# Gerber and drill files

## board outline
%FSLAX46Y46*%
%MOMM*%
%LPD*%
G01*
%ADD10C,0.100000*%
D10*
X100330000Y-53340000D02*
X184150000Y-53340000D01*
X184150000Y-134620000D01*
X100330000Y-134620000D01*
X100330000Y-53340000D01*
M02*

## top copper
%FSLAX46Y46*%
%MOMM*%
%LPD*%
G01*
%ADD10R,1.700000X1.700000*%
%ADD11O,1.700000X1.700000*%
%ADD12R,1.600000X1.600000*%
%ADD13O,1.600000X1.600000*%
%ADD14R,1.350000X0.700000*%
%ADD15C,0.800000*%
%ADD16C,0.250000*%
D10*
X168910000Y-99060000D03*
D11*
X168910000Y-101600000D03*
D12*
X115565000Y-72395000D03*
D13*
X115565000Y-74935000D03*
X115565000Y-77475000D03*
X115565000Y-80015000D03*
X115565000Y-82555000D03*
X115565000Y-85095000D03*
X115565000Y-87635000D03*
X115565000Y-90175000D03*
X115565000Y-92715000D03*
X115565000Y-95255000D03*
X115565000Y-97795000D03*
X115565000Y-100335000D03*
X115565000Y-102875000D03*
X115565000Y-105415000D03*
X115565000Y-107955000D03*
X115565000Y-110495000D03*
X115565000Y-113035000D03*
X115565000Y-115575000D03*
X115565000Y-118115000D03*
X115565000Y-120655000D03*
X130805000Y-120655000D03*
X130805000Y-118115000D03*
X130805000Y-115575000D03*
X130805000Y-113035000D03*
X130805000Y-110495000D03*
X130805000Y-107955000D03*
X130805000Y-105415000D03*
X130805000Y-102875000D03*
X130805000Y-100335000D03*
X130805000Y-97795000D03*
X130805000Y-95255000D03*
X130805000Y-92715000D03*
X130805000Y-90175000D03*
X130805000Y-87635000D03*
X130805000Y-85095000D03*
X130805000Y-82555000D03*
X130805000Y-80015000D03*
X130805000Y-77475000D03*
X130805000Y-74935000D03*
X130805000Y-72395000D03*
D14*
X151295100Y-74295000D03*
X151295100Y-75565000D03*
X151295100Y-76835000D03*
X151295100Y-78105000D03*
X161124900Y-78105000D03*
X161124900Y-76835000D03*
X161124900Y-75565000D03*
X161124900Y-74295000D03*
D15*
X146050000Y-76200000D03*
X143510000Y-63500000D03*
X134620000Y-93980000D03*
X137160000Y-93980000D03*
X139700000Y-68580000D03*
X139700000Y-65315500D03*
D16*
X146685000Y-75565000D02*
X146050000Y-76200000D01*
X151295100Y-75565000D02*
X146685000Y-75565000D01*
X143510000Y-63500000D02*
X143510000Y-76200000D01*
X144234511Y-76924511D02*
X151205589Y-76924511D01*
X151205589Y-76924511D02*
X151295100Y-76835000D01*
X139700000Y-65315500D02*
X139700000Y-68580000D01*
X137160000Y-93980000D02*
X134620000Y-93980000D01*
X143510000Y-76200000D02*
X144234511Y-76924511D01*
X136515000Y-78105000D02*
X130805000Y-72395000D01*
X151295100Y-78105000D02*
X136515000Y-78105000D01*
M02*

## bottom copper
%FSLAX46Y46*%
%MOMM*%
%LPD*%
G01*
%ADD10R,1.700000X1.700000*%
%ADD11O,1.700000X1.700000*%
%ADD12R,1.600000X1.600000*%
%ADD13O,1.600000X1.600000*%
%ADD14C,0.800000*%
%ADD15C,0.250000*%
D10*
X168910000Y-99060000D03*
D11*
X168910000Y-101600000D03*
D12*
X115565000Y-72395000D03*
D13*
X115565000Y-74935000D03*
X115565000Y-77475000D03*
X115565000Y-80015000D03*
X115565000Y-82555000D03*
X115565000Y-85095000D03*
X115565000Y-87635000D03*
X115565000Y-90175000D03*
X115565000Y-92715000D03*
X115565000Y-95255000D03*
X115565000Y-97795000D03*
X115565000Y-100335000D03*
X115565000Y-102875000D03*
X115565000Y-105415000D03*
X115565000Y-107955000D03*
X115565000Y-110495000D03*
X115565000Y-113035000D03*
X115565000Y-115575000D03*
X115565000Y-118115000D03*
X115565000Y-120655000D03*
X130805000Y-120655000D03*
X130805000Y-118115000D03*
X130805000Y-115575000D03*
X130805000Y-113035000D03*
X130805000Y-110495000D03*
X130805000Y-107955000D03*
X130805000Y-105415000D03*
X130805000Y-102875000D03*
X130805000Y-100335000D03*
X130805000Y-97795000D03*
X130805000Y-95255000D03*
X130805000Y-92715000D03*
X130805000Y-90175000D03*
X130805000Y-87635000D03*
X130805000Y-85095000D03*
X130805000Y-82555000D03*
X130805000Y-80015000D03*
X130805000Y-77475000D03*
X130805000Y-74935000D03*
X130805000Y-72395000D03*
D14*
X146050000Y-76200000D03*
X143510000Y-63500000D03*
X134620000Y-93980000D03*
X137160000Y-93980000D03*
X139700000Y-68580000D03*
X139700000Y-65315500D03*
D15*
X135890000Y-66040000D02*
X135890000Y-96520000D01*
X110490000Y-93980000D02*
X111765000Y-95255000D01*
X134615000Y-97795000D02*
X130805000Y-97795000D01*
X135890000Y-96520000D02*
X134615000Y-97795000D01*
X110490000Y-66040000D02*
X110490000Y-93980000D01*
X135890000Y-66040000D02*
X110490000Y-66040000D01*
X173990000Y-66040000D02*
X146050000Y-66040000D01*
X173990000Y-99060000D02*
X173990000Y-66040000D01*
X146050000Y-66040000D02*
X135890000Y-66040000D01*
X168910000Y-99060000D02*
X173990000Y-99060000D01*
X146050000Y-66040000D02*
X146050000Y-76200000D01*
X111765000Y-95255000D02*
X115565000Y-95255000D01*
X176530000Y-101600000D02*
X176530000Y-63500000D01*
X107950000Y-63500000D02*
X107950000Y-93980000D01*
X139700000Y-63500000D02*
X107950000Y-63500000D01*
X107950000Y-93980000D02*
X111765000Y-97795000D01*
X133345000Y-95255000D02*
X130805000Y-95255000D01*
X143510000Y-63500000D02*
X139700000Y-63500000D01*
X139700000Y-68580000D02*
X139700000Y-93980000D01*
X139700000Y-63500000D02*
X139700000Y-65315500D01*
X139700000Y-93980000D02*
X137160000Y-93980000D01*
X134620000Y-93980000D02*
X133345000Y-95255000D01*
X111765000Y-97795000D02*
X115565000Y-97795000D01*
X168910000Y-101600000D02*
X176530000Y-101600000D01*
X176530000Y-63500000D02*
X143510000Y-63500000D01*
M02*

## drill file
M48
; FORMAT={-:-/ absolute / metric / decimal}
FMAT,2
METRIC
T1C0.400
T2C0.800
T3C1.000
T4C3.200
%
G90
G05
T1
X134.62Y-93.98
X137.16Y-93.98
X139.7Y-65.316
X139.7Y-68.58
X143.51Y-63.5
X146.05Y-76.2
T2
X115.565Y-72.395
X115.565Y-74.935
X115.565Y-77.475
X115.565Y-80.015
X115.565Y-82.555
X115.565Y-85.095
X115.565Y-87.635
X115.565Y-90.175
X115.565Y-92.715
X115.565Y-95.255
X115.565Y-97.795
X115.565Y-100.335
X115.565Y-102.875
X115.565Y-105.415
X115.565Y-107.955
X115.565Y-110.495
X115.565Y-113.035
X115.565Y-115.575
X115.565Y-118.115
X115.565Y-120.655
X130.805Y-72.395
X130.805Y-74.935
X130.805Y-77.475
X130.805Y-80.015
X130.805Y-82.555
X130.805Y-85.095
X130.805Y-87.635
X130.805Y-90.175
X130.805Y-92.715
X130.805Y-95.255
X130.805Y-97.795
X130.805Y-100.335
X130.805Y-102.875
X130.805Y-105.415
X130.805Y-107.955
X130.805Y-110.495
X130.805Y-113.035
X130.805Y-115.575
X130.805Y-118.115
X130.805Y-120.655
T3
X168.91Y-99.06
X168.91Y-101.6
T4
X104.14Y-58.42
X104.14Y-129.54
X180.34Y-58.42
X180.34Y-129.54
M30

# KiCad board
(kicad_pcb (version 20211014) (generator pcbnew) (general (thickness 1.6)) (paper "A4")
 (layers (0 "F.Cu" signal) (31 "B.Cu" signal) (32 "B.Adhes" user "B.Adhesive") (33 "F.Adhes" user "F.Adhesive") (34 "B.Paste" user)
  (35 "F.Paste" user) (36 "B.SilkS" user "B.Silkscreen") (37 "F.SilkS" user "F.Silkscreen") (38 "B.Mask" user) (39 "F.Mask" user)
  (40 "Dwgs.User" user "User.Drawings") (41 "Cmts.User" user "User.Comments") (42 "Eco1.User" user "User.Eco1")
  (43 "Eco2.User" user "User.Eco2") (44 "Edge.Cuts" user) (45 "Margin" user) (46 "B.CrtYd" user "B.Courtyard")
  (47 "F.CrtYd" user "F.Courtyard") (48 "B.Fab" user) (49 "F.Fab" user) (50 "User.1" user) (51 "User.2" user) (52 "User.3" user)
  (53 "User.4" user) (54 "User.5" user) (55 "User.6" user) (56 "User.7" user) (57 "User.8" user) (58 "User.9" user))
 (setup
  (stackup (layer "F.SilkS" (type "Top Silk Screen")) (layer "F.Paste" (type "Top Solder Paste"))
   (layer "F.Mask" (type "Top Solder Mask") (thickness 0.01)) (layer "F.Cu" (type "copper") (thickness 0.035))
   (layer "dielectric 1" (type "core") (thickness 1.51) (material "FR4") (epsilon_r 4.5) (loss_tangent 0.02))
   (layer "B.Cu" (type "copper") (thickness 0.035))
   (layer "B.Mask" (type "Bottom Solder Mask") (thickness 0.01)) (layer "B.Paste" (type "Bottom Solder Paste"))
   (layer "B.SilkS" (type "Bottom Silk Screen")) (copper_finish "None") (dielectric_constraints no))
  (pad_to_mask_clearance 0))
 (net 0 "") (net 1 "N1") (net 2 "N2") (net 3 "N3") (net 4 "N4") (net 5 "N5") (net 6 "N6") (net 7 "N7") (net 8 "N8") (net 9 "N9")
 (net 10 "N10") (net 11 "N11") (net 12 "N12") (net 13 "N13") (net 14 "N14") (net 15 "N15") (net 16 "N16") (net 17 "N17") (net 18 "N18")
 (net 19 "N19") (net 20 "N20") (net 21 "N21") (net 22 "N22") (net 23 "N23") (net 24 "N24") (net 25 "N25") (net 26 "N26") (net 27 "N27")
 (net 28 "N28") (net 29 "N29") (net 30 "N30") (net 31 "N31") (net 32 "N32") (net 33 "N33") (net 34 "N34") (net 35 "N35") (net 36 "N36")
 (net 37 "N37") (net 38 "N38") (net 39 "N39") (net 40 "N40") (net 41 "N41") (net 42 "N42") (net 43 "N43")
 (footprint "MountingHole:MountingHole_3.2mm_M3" (layer "F.Cu") (at 180.34 129.54)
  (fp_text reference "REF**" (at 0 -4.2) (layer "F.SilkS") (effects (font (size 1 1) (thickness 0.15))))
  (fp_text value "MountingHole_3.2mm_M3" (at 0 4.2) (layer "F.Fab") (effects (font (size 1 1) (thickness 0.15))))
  (pad "" np_thru_hole circle (at 0 0) (size 3.2 3.2) (drill 3.2) (layers *.Cu *.Mask)))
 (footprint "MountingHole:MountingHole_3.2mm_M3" (layer "F.Cu") (at 104.14 58.42)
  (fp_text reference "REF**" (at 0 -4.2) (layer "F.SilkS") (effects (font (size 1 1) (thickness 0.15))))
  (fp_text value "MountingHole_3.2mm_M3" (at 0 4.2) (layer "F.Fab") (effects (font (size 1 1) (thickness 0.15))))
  (pad "" np_thru_hole circle (at 0 0) (size 3.2 3.2) (drill 3.2) (layers *.Cu *.Mask)))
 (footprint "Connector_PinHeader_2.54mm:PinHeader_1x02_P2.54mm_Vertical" (layer "F.Cu") (at 168.91 99.06)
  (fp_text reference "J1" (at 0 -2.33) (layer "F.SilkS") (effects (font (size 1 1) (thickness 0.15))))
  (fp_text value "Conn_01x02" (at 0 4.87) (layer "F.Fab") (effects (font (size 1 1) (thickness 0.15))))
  (pad "1" thru_hole rect (at 0 0) (size 1.7 1.7) (drill 1) (layers *.Cu *.Mask) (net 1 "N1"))
  (pad "2" thru_hole oval (at 0 2.54) (size 1.7 1.7) (drill 1) (layers *.Cu *.Mask) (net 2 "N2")))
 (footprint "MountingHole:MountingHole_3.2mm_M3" (layer "F.Cu") (at 180.34 58.42)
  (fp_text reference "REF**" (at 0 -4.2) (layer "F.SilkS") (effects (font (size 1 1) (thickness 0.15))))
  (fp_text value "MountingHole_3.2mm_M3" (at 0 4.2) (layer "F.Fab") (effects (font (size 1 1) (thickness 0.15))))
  (pad "" np_thru_hole circle (at 0 0) (size 3.2 3.2) (drill 3.2) (layers *.Cu *.Mask)))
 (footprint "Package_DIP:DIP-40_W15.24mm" (layer "F.Cu") (at 115.565 72.395)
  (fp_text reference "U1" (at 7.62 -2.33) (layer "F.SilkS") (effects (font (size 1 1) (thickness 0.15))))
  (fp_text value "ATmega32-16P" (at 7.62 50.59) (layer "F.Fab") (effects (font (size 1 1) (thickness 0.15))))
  (pad "1" thru_hole rect (at 0 0) (size 1.6 1.6) (drill 0.8) (layers *.Cu *.Mask) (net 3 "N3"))
  (pad "2" thru_hole oval (at 0 2.54) (size 1.6 1.6) (drill 0.8) (layers *.Cu *.Mask) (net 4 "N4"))
  (pad "3" thru_hole oval (at 0 5.08) (size 1.6 1.6) (drill 0.8) (layers *.Cu *.Mask) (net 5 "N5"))
  (pad "4" thru_hole oval (at 0 7.62) (size 1.6 1.6) (drill 0.8) (layers *.Cu *.Mask) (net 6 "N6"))
  (pad "5" thru_hole oval (at 0 10.16) (size 1.6 1.6) (drill 0.8) (layers *.Cu *.Mask) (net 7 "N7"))
  (pad "6" thru_hole oval (at 0 12.7) (size 1.6 1.6) (drill 0.8) (layers *.Cu *.Mask) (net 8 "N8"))
  (pad "7" thru_hole oval (at 0 15.24) (size 1.6 1.6) (drill 0.8) (layers *.Cu *.Mask) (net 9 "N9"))
  (pad "8" thru_hole oval (at 0 17.78) (size 1.6 1.6) (drill 0.8) (layers *.Cu *.Mask) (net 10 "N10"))
  (pad "9" thru_hole oval (at 0 20.32) (size 1.6 1.6) (drill 0.8) (layers *.Cu *.Mask) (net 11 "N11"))
  (pad "10" thru_hole oval (at 0 22.86) (size 1.6 1.6) (drill 0.8) (layers *.Cu *.Mask) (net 1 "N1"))
  (pad "11" thru_hole oval (at 0 25.4) (size 1.6 1.6) (drill 0.8) (layers *.Cu *.Mask) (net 2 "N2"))
  (pad "12" thru_hole oval (at 0 27.94) (size 1.6 1.6) (drill 0.8) (layers *.Cu *.Mask) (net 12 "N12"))
  (pad "13" thru_hole oval (at 0 30.48) (size 1.6 1.6) (drill 0.8) (layers *.Cu *.Mask) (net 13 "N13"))
  (pad "14" thru_hole oval (at 0 33.02) (size 1.6 1.6) (drill 0.8) (layers *.Cu *.Mask) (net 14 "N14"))
  (pad "15" thru_hole oval (at 0 35.56) (size 1.6 1.6) (drill 0.8) (layers *.Cu *.Mask) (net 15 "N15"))
  (pad "16" thru_hole oval (at 0 38.1) (size 1.6 1.6) (drill 0.8) (layers *.Cu *.Mask) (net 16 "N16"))
  (pad "17" thru_hole oval (at 0 40.64) (size 1.6 1.6) (drill 0.8) (layers *.Cu *.Mask) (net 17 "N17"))
  (pad "18" thru_hole oval (at 0 43.18) (size 1.6 1.6) (drill 0.8) (layers *.Cu *.Mask) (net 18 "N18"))
  (pad "19" thru_hole oval (at 0 45.72) (size 1.6 1.6) (drill 0.8) (layers *.Cu *.Mask) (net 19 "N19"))
  (pad "20" thru_hole oval (at 0 48.26) (size 1.6 1.6) (drill 0.8) (layers *.Cu *.Mask) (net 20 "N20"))
  (pad "21" thru_hole oval (at 15.24 48.26) (size 1.6 1.6) (drill 0.8) (layers *.Cu *.Mask) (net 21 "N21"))
  (pad "22" thru_hole oval (at 15.24 45.72) (size 1.6 1.6) (drill 0.8) (layers *.Cu *.Mask) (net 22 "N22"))
  (pad "23" thru_hole oval (at 15.24 43.18) (size 1.6 1.6) (drill 0.8) (layers *.Cu *.Mask) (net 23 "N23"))
  (pad "24" thru_hole oval (at 15.24 40.64) (size 1.6 1.6) (drill 0.8) (layers *.Cu *.Mask) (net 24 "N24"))
  (pad "25" thru_hole oval (at 15.24 38.1) (size 1.6 1.6) (drill 0.8) (layers *.Cu *.Mask) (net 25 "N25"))
  (pad "26" thru_hole oval (at 15.24 35.56) (size 1.6 1.6) (drill 0.8) (layers *.Cu *.Mask) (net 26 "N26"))
  (pad "27" thru_hole oval (at 15.24 33.02) (size 1.6 1.6) (drill 0.8) (layers *.Cu *.Mask) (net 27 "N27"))
  (pad "28" thru_hole oval (at 15.24 30.48) (size 1.6 1.6) (drill 0.8) (layers *.Cu *.Mask) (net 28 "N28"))
  (pad "29" thru_hole oval (at 15.24 27.94) (size 1.6 1.6) (drill 0.8) (layers *.Cu *.Mask) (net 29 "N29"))
  (pad "30" thru_hole oval (at 15.24 25.4) (size 1.6 1.6) (drill 0.8) (layers *.Cu *.Mask) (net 1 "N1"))
  (pad "31" thru_hole oval (at 15.24 22.86) (size 1.6 1.6) (drill 0.8) (layers *.Cu *.Mask) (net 2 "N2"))
  (pad "32" thru_hole oval (at 15.24 20.32) (size 1.6 1.6) (drill 0.8) (layers *.Cu *.Mask) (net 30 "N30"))
  (pad "33" thru_hole oval (at 15.24 17.78) (size 1.6 1.6) (drill 0.8) (layers *.Cu *.Mask) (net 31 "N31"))
  (pad "34" thru_hole oval (at 15.24 15.24) (size 1.6 1.6) (drill 0.8) (layers *.Cu *.Mask) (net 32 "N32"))
  (pad "35" thru_hole oval (at 15.24 12.7) (size 1.6 1.6) (drill 0.8) (layers *.Cu *.Mask) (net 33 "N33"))
  (pad "36" thru_hole oval (at 15.24 10.16) (size 1.6 1.6) (drill 0.8) (layers *.Cu *.Mask) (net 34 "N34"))
  (pad "37" thru_hole oval (at 15.24 7.62) (size 1.6 1.6) (drill 0.8) (layers *.Cu *.Mask) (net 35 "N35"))
  (pad "38" thru_hole oval (at 15.24 5.08) (size 1.6 1.6) (drill 0.8) (layers *.Cu *.Mask) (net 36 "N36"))
  (pad "39" thru_hole oval (at 15.24 2.54) (size 1.6 1.6) (drill 0.8) (layers *.Cu *.Mask) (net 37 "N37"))
  (pad "40" thru_hole oval (at 15.24 0) (size 1.6 1.6) (drill 0.8) (layers *.Cu *.Mask) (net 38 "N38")))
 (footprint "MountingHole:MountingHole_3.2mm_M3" (layer "F.Cu") (at 104.14 129.54)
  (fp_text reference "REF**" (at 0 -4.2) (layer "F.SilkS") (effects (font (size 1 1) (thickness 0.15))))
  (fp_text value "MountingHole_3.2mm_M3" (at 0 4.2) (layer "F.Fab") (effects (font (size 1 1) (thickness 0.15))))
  (pad "" np_thru_hole circle (at 0 0) (size 3.2 3.2) (drill 3.2) (layers *.Cu *.Mask)))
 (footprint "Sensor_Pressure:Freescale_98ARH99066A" (layer "F.Cu") (at 156.21 76.2)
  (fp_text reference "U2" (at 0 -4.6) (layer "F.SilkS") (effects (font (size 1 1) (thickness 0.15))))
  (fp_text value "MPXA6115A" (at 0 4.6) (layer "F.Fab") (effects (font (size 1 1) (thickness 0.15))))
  (pad "1" smd rect (at -4.9149 -1.905) (size 1.35 0.7) (layers "F.Cu" "F.Paste" "F.Mask") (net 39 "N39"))
  (pad "2" smd rect (at -4.9149 -0.635) (size 1.35 0.7) (layers "F.Cu" "F.Paste" "F.Mask") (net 1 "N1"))
  (pad "3" smd rect (at -4.9149 0.635) (size 1.35 0.7) (layers "F.Cu" "F.Paste" "F.Mask") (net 2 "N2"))
  (pad "4" smd rect (at -4.9149 1.905) (size 1.35 0.7) (layers "F.Cu" "F.Paste" "F.Mask") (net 38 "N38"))
  (pad "5" smd rect (at 4.9149 1.905) (size 1.35 0.7) (layers "F.Cu" "F.Paste" "F.Mask") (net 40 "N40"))
  (pad "6" smd rect (at 4.9149 0.635) (size 1.35 0.7) (layers "F.Cu" "F.Paste" "F.Mask") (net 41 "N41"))
  (pad "7" smd rect (at 4.9149 -0.635) (size 1.35 0.7) (layers "F.Cu" "F.Paste" "F.Mask") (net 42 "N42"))
  (pad "8" smd rect (at 4.9149 -1.905) (size 1.35 0.7) (layers "F.Cu" "F.Paste" "F.Mask") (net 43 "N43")))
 (gr_rect (start 100.33 53.34) (end 184.15 134.62) (layer "Edge.Cuts") (width 0.1) (fill none))
 (segment (start 146.685 75.565) (end 146.05 76.2) (width 0.25) (layer "F.Cu") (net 1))
 (segment (start 151.2951 75.565) (end 146.685 75.565) (width 0.25) (layer "F.Cu") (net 1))
 (via (at 146.05 76.2) (size 0.8) (drill 0.4) (layers "F.Cu" "B.Cu") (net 1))
 (segment (start 135.89 66.04) (end 135.89 96.52) (width 0.25) (layer "B.Cu") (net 1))
 (segment (start 110.49 93.98) (end 111.765 95.255) (width 0.25) (layer "B.Cu") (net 1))
 (segment (start 134.615 97.795) (end 130.805 97.795) (width 0.25) (layer "B.Cu") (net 1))
 (segment (start 135.89 96.52) (end 134.615 97.795) (width 0.25) (layer "B.Cu") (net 1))
 (segment (start 110.49 66.04) (end 110.49 93.98) (width 0.25) (layer "B.Cu") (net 1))
 (segment (start 135.89 66.04) (end 110.49 66.04) (width 0.25) (layer "B.Cu") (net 1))
 (segment (start 173.99 66.04) (end 146.05 66.04) (width 0.25) (layer "B.Cu") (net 1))
 (segment (start 173.99 99.06) (end 173.99 66.04) (width 0.25) (layer "B.Cu") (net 1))
 (segment (start 146.05 66.04) (end 135.89 66.04) (width 0.25) (layer "B.Cu") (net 1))
 (segment (start 168.91 99.06) (end 173.99 99.06) (width 0.25) (layer "B.Cu") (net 1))
 (segment (start 146.05 66.04) (end 146.05 76.2) (width 0.25) (layer "B.Cu") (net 1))
 (segment (start 111.765 95.255) (end 115.565 95.255) (width 0.25) (layer "B.Cu") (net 1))
 (segment (start 143.51 63.5) (end 143.51 76.2) (width 0.25) (layer "F.Cu") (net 2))
 (segment (start 144.234511 76.924511) (end 151.205589 76.924511) (width 0.25) (layer "F.Cu") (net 2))
 (segment (start 151.205589 76.924511) (end 151.2951 76.835) (width 0.25) (layer "F.Cu") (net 2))
 (segment (start 139.7 65.3155) (end 139.7 68.58) (width 0.25) (layer "F.Cu") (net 2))
 (segment (start 137.16 93.98) (end 134.62 93.98) (width 0.25) (layer "F.Cu") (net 2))
 (segment (start 143.51 76.2) (end 144.234511 76.924511) (width 0.25) (layer "F.Cu") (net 2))
 (via (at 143.51 63.5) (size 0.8) (drill 0.4) (layers "F.Cu" "B.Cu") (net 2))
 (via (at 134.62 93.98) (size 0.8) (drill 0.4) (layers "F.Cu" "B.Cu") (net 2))
 (via (at 137.16 93.98) (size 0.8) (drill 0.4) (layers "F.Cu" "B.Cu") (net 2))
 (via (at 139.7 68.58) (size 0.8) (drill 0.4) (layers "F.Cu" "B.Cu") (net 2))
 (via (at 139.7 65.3155) (size 0.8) (drill 0.4) (layers "F.Cu" "B.Cu") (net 2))
 (segment (start 176.53 101.6) (end 176.53 63.5) (width 0.25) (layer "B.Cu") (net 2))
 (segment (start 107.95 63.5) (end 107.95 93.98) (width 0.25) (layer "B.Cu") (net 2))
 (segment (start 139.7 63.5) (end 107.95 63.5) (width 0.25) (layer "B.Cu") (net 2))
 (segment (start 107.95 93.98) (end 111.765 97.795) (width 0.25) (layer "B.Cu") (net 2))
 (segment (start 133.345 95.255) (end 130.805 95.255) (width 0.25) (layer "B.Cu") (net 2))
 (segment (start 143.51 63.5) (end 139.7 63.5) (width 0.25) (layer "B.Cu") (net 2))
 (segment (start 139.7 68.58) (end 139.7 93.98) (width 0.25) (layer "B.Cu") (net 2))
 (segment (start 139.7 63.5) (end 139.7 65.3155) (width 0.25) (layer "B.Cu") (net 2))
 (segment (start 139.7 93.98) (end 137.16 93.98) (width 0.25) (layer "B.Cu") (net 2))
 (segment (start 134.62 93.98) (end 133.345 95.255) (width 0.25) (layer "B.Cu") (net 2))
 (segment (start 111.765 97.795) (end 115.565 97.795) (width 0.25) (layer "B.Cu") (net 2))
 (segment (start 168.91 101.6) (end 176.53 101.6) (width 0.25) (layer "B.Cu") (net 2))
 (segment (start 176.53 63.5) (end 143.51 63.5) (width 0.25) (layer "B.Cu") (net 2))
 (segment (start 136.515 78.105) (end 130.805 72.395) (width 0.25) (layer "F.Cu") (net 38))
 (segment (start 151.2951 78.105) (end 136.515 78.105) (width 0.25) (layer "F.Cu") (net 38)))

